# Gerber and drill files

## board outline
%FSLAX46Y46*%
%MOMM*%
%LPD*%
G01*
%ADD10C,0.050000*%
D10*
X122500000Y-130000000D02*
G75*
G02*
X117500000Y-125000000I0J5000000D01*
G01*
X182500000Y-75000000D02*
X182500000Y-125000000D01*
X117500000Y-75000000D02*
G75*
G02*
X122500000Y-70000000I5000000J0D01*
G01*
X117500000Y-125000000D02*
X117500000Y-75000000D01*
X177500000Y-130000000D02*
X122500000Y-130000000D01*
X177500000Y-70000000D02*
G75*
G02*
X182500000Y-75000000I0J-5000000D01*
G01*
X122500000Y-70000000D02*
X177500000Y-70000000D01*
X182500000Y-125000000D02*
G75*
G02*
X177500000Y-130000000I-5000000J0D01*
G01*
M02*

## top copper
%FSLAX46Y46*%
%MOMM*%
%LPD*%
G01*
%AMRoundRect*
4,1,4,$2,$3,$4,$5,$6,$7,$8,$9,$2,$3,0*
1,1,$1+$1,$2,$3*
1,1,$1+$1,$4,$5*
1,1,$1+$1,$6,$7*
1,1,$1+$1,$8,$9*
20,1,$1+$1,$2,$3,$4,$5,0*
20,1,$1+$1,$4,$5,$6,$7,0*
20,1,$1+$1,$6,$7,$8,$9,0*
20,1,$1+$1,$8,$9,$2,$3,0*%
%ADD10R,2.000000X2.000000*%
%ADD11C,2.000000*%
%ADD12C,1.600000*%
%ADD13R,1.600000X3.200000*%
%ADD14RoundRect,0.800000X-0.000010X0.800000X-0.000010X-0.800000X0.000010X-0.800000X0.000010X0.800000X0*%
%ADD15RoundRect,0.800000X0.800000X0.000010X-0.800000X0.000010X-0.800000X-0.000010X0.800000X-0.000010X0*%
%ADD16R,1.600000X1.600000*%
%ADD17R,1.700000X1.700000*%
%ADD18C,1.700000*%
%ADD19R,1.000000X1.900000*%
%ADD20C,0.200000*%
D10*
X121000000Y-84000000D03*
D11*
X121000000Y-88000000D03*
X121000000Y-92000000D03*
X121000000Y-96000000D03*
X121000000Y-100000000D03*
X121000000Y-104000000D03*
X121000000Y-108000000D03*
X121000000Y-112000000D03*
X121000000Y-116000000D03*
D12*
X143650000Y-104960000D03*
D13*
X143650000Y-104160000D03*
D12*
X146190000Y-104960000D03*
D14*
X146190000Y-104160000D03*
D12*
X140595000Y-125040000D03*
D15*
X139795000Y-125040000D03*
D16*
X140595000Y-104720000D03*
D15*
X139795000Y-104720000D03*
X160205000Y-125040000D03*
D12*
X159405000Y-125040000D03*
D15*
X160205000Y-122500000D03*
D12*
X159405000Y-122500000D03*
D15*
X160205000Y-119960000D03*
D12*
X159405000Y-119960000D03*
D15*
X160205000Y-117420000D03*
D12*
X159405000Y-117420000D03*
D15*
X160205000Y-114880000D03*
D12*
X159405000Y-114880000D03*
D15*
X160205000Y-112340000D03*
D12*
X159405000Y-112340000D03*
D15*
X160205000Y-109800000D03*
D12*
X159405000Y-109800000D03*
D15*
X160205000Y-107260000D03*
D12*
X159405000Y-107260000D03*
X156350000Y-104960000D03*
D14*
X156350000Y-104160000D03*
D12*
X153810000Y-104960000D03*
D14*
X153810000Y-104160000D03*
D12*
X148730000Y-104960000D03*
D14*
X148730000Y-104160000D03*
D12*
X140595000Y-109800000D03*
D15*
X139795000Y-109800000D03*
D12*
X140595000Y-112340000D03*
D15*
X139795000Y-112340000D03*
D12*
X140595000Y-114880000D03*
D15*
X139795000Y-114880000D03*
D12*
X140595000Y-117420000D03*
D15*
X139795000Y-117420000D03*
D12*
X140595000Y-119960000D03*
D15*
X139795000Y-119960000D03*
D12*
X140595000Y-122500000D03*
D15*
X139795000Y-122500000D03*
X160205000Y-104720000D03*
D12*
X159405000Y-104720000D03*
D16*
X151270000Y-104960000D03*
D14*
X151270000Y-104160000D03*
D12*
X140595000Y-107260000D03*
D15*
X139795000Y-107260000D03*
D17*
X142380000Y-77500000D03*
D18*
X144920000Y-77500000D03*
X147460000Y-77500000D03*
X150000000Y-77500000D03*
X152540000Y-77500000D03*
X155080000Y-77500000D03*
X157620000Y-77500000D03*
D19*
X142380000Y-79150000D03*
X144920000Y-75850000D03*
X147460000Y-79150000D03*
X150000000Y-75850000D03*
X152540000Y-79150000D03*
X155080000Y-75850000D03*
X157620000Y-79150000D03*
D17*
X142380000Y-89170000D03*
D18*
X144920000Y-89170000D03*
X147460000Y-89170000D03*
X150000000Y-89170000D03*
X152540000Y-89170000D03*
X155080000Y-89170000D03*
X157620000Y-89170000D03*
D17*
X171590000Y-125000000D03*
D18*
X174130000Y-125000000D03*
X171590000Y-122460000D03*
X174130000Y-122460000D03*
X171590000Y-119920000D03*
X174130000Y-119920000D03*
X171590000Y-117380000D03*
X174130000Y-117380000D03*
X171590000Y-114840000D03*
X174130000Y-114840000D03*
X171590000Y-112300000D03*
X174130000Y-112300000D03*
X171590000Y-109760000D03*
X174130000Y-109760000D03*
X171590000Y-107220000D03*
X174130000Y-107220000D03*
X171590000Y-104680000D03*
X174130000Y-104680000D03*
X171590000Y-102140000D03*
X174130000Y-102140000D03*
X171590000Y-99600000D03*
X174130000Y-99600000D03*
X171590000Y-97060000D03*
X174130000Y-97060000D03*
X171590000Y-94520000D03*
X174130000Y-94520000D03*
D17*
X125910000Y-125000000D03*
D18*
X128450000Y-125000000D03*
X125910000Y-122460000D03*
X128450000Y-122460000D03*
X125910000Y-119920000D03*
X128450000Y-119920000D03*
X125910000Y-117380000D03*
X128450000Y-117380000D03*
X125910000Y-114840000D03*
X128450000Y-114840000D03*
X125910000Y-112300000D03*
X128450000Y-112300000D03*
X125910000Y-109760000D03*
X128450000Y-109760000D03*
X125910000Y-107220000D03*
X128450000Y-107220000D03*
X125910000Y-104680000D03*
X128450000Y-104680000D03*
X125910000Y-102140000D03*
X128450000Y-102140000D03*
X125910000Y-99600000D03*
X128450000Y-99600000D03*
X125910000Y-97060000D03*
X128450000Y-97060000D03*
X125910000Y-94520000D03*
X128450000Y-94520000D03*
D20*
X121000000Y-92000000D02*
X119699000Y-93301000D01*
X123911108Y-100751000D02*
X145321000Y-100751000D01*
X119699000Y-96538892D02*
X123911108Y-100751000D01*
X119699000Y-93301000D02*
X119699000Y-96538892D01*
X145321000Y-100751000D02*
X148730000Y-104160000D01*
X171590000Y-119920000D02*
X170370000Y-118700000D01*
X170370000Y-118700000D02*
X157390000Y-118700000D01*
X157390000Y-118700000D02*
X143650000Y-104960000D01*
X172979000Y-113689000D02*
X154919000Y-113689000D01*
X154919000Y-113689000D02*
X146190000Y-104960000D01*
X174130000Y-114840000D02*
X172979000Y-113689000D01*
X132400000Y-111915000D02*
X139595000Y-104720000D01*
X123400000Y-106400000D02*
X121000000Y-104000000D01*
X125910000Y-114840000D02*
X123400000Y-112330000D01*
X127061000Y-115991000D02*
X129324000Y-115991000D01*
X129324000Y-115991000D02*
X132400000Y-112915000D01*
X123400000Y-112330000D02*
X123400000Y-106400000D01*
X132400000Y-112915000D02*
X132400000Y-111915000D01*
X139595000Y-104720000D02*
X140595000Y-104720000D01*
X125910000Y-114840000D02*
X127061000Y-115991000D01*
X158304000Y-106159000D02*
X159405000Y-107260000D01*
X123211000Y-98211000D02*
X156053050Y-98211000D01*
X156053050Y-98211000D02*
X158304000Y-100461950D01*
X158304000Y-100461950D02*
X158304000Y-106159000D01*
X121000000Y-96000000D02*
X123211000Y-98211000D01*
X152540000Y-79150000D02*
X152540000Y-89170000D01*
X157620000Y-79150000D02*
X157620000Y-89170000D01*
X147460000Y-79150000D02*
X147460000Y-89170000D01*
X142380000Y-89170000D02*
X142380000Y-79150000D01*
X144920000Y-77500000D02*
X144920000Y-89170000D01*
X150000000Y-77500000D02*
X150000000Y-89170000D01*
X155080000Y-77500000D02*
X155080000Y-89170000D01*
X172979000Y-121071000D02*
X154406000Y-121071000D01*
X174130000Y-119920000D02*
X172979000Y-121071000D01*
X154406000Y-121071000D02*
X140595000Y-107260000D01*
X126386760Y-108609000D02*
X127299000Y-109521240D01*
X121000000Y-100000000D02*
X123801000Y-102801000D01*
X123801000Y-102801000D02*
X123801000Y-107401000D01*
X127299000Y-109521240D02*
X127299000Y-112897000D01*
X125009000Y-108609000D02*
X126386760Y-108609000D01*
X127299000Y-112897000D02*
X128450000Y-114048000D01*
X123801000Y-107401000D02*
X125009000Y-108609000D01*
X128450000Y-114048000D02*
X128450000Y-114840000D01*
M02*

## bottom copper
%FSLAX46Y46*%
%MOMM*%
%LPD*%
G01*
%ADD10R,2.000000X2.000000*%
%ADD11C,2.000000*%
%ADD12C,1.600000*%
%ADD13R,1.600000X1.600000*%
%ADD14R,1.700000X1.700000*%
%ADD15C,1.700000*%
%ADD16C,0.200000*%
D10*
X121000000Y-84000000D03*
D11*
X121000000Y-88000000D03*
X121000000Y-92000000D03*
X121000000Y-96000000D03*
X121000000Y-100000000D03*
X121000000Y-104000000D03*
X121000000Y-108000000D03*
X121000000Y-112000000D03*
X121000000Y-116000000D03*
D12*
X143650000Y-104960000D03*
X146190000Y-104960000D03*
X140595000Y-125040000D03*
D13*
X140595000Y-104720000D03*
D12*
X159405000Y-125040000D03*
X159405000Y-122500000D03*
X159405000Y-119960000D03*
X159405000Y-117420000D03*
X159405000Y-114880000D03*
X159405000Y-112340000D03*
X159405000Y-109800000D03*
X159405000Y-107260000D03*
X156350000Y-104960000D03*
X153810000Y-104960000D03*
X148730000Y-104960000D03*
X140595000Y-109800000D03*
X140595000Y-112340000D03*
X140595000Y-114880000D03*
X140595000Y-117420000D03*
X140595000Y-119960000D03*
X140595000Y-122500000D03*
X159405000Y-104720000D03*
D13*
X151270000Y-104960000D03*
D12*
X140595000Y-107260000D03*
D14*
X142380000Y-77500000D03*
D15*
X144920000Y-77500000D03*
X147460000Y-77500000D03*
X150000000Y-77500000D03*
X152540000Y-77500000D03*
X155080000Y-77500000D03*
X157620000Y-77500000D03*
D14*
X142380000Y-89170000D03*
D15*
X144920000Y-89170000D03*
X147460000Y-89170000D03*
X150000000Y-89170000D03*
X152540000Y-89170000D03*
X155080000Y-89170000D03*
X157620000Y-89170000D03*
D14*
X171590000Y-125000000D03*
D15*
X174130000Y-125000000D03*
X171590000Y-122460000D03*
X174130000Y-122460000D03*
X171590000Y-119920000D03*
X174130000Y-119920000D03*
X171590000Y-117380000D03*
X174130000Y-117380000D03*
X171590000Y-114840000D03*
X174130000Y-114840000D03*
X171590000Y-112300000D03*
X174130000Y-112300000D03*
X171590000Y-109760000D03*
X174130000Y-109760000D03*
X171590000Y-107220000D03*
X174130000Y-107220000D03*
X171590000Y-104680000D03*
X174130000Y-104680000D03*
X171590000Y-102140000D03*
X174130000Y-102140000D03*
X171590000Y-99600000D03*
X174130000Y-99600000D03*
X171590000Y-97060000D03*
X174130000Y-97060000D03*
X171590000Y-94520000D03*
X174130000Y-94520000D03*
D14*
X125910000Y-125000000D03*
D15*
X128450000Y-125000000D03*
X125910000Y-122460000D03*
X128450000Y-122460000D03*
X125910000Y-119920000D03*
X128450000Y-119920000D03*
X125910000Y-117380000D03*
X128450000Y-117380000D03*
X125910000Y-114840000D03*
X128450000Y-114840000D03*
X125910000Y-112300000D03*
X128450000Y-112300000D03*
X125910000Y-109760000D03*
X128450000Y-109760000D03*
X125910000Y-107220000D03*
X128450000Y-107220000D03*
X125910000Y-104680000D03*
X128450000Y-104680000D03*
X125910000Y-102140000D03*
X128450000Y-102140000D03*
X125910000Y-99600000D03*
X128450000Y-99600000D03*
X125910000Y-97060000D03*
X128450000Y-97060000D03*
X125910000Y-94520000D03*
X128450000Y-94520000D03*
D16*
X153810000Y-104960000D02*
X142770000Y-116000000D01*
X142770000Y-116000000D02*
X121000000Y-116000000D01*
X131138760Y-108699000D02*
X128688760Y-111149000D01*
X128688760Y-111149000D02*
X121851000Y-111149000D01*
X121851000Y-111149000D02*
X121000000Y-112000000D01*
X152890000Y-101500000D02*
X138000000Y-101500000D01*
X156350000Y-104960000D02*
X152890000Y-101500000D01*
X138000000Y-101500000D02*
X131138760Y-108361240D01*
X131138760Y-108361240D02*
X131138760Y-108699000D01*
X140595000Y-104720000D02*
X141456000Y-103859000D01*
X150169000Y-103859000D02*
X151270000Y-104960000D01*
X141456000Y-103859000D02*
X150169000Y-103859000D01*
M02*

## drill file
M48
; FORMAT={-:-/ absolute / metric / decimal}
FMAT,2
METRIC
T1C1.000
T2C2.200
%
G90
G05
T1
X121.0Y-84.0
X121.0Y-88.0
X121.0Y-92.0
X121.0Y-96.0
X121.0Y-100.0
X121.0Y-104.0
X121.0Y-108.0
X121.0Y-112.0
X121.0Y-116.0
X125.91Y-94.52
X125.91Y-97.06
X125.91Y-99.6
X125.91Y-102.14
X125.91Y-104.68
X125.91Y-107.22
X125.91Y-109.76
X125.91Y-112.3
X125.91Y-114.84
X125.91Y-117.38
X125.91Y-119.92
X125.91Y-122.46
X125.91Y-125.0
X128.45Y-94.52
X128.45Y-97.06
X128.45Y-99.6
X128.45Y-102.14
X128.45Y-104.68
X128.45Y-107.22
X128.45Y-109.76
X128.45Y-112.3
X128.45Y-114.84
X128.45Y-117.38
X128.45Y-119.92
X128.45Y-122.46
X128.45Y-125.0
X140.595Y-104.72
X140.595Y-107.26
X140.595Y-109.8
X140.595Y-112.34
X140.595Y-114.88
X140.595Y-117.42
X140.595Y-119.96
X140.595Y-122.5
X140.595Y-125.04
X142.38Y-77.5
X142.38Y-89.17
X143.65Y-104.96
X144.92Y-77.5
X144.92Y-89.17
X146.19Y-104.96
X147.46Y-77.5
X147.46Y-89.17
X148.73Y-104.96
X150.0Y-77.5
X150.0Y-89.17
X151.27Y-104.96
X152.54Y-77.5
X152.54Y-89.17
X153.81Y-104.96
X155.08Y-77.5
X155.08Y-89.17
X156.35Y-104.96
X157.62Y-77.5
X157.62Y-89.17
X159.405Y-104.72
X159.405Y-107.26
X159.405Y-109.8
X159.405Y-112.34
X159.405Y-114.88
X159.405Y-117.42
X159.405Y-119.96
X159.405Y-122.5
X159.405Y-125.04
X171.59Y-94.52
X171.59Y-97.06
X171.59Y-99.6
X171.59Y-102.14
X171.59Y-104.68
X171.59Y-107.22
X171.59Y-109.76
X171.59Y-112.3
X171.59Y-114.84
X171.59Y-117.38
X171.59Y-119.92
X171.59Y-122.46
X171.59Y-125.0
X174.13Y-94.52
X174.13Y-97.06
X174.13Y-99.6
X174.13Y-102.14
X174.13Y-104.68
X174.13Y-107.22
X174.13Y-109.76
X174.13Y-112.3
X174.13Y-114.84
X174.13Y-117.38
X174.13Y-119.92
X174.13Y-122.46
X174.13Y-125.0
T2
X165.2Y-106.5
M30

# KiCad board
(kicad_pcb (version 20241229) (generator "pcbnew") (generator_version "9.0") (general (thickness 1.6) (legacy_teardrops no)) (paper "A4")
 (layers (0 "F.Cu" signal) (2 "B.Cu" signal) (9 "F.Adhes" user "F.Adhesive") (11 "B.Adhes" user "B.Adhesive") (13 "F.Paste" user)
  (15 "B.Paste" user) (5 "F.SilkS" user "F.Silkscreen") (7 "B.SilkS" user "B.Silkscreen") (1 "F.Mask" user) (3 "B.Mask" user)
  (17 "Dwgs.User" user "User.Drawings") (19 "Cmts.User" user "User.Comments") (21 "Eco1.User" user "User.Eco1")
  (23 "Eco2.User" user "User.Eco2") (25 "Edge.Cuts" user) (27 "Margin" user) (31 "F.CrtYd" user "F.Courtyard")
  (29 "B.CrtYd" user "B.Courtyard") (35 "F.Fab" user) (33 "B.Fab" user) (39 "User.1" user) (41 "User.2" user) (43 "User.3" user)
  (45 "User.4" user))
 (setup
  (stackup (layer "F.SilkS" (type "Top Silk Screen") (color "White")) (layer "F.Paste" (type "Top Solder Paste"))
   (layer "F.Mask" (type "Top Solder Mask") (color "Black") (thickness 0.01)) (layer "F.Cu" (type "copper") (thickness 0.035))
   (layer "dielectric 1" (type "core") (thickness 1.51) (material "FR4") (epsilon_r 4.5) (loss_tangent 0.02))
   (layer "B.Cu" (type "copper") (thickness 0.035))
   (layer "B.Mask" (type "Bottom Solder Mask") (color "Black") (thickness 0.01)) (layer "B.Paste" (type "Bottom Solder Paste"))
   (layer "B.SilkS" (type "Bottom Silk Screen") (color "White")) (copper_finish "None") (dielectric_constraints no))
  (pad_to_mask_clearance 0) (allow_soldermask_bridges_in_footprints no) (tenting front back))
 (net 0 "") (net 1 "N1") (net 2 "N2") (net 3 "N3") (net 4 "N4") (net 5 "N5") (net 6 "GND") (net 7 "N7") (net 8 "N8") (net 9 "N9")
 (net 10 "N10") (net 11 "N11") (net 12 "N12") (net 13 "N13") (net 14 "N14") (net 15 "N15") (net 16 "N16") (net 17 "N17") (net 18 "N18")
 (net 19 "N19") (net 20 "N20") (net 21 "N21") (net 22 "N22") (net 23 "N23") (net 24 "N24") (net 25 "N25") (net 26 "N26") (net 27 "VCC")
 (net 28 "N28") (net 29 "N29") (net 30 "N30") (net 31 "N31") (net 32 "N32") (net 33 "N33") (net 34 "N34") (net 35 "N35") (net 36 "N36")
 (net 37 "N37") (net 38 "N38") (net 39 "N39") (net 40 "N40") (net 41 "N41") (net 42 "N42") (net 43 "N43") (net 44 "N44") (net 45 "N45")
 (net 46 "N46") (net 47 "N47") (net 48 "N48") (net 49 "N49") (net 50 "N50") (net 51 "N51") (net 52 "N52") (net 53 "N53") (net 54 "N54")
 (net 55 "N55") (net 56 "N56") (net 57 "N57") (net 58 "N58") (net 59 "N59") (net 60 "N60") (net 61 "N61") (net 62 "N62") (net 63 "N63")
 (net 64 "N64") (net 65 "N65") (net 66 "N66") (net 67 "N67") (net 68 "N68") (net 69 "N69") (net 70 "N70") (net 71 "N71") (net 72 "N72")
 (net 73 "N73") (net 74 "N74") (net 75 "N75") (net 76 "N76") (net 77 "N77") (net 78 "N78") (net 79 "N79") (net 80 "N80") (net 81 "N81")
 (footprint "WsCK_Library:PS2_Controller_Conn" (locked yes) (layer "F.Cu") (at 121 100)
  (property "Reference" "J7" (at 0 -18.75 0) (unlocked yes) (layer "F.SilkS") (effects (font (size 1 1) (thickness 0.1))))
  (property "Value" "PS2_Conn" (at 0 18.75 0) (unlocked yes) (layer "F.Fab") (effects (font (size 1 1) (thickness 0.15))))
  (pad "1" thru_hole rect (at 0 -16 270) (size 2 2) (drill 1) (layers "*.Cu" "*.Mask") (remove_unused_layers no) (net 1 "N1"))
  (pad "2" thru_hole circle (at 0 -12 270) (size 2 2) (drill 1) (layers "*.Cu" "*.Mask") (remove_unused_layers no) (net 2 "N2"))
  (pad "3" thru_hole circle (at 0 -8 270) (size 2 2) (drill 1) (layers "*.Cu" "*.Mask") (remove_unused_layers no) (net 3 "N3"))
  (pad "4" thru_hole circle (at 0 -4 270) (size 2 2) (drill 1) (layers "*.Cu" "*.Mask") (remove_unused_layers no) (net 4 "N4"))
  (pad "5" thru_hole circle (at 0 0 270) (size 2 2) (drill 1) (layers "*.Cu" "*.Mask") (remove_unused_layers no) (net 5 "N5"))
  (pad "6" thru_hole circle (at 0 4 270) (size 2 2) (drill 1) (layers "*.Cu" "*.Mask") (remove_unused_layers no) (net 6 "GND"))
  (pad "7" thru_hole circle (at 0 8 270) (size 2 2) (drill 1) (layers "*.Cu" "*.Mask") (remove_unused_layers no) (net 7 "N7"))
  (pad "8" thru_hole circle (at 0 12 270) (size 2 2) (drill 1) (layers "*.Cu" "*.Mask") (remove_unused_layers no) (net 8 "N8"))
  (pad "9" thru_hole circle (at 0 16 270) (size 2 2) (drill 1) (layers "*.Cu" "*.Mask") (remove_unused_layers no) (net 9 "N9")))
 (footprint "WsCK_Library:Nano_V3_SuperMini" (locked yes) (layer "F.Cu") (at 150 116.66 180)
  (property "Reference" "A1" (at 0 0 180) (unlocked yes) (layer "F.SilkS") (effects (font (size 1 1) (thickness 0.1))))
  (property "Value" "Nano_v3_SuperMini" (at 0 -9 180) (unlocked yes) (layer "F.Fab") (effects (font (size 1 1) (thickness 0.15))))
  (pad "1" thru_hole circle (at 6.35 11.7 180) (size 1.6 1.6) (drill 1) (layers "*.Cu" "*.Mask") (remove_unused_layers no) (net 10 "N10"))
  (pad "1" smd rect (at 6.35 12.5 270) (size 3.2 1.6) (layers "F.Cu" "F.Mask") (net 10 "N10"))
  (pad "2" thru_hole circle (at 3.81 11.7 180) (size 1.6 1.6) (drill 1) (layers "*.Cu" "*.Mask") (remove_unused_layers no) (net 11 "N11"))
  (pad "2" smd roundrect (at 3.81 12.5 270) (size 3.2 1.6) (layers "F.Cu" "F.Mask") (roundrect_rratio 0.5) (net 11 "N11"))
  (pad "3" thru_hole circle (at 9.405 -8.38 180) (size 1.6 1.6) (drill 1) (layers "*.Cu" "*.Mask") (remove_unused_layers no) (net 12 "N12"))
  (pad "3" smd roundrect (at 10.205 -8.38 180) (size 3.2 1.6) (layers "F.Cu" "F.Mask") (roundrect_rratio 0.5) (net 12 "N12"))
  (pad "4" thru_hole rect (at 9.405 11.94 180) (size 1.6 1.6) (drill 1) (layers "*.Cu" "*.Mask") (remove_unused_layers no) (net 6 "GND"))
  (pad "4" smd roundrect (at 10.205 11.94 180) (size 3.2 1.6) (layers "F.Cu" "F.Mask") (roundrect_rratio 0.5) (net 6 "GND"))
  (pad "6" smd roundrect (at -10.205 -8.38 180) (size 3.2 1.6) (layers "F.Cu" "F.Mask") (roundrect_rratio 0.5) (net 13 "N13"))
  (pad "6" thru_hole circle (at -9.405 -8.38 180) (size 1.6 1.6) (drill 1) (layers "*.Cu" "*.Mask") (remove_unused_layers no) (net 13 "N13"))
  (pad "7" smd roundrect (at -10.205 -5.84 180) (size 3.2 1.6) (layers "F.Cu" "F.Mask") (roundrect_rratio 0.5) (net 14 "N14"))
  (pad "7" thru_hole circle (at -9.405 -5.84 180) (size 1.6 1.6) (drill 1) (layers "*.Cu" "*.Mask") (remove_unused_layers no) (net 14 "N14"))
  (pad "8" smd roundrect (at -10.205 -3.3 180) (size 3.2 1.6) (layers "F.Cu" "F.Mask") (roundrect_rratio 0.5) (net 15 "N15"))
  (pad "8" thru_hole circle (at -9.405 -3.3 180) (size 1.6 1.6) (drill 1) (layers "*.Cu" "*.Mask") (remove_unused_layers no) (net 15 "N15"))
  (pad "9" smd roundrect (at -10.205 -0.76 180) (size 3.2 1.6) (layers "F.Cu" "F.Mask") (roundrect_rratio 0.5) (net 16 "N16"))
  (pad "9" thru_hole circle (at -9.405 -0.76 180) (size 1.6 1.6) (drill 1) (layers "*.Cu" "*.Mask") (remove_unused_layers no) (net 16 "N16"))
  (pad "10" smd roundrect (at -10.205 1.78 180) (size 3.2 1.6) (layers "F.Cu" "F.Mask") (roundrect_rratio 0.5) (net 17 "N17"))
  (pad "10" thru_hole circle (at -9.405 1.78 180) (size 1.6 1.6) (drill 1) (layers "*.Cu" "*.Mask") (remove_unused_layers no) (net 17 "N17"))
  (pad "11" smd roundrect (at -10.205 4.32 180) (size 3.2 1.6) (layers "F.Cu" "F.Mask") (roundrect_rratio 0.5) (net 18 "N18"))
  (pad "11" thru_hole circle (at -9.405 4.32 180) (size 1.6 1.6) (drill 1) (layers "*.Cu" "*.Mask") (remove_unused_layers no) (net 18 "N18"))
  (pad "12" smd roundrect (at -10.205 6.86 180) (size 3.2 1.6) (layers "F.Cu" "F.Mask") (roundrect_rratio 0.5) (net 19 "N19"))
  (pad "12" thru_hole circle (at -9.405 6.86 180) (size 1.6 1.6) (drill 1) (layers "*.Cu" "*.Mask") (remove_unused_layers no) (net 19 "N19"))
  (pad "13" smd roundrect (at -10.205 9.4 180) (size 3.2 1.6) (layers "F.Cu" "F.Mask") (roundrect_rratio 0.5) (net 4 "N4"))
  (pad "13" thru_hole circle (at -9.405 9.4 180) (size 1.6 1.6) (drill 1) (layers "*.Cu" "*.Mask") (remove_unused_layers no) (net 4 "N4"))
  (pad "14" thru_hole circle (at -6.35 11.7 180) (size 1.6 1.6) (drill 1) (layers "*.Cu" "*.Mask") (remove_unused_layers no) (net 8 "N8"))
  (pad "14" smd roundrect (at -6.35 12.5 270) (size 3.2 1.6) (layers "F.Cu" "F.Mask") (roundrect_rratio 0.5) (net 8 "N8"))
  (pad "15" thru_hole circle (at -3.81 11.7 180) (size 1.6 1.6) (drill 1) (layers "*.Cu" "*.Mask") (remove_unused_layers no) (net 9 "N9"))
  (pad "15" smd roundrect (at -3.81 12.5 270) (size 3.2 1.6) (layers "F.Cu" "F.Mask") (roundrect_rratio 0.5) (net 9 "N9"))
  (pad "16" thru_hole circle (at 1.27 11.7 180) (size 1.6 1.6) (drill 1) (layers "*.Cu" "*.Mask") (remove_unused_layers no) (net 3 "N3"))
  (pad "16" smd roundrect (at 1.27 12.5 270) (size 3.2 1.6) (layers "F.Cu" "F.Mask") (roundrect_rratio 0.5) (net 3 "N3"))
  (pad "19" thru_hole circle (at 9.405 6.86 180) (size 1.6 1.6) (drill 1) (layers "*.Cu" "*.Mask") (remove_unused_layers no) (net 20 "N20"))
  (pad "19" smd roundrect (at 10.205 6.86 180) (size 3.2 1.6) (layers "F.Cu" "F.Mask") (roundrect_rratio 0.5) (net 20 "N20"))
  (pad "20" thru_hole circle (at 9.405 4.32 180) (size 1.6 1.6) (drill 1) (layers "*.Cu" "*.Mask") (remove_unused_layers no) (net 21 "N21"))
  (pad "20" smd roundrect (at 10.205 4.32 180) (size 3.2 1.6) (layers "F.Cu" "F.Mask") (roundrect_rratio 0.5) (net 21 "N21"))
  (pad "21" thru_hole circle (at 9.405 1.78 180) (size 1.6 1.6) (drill 1) (layers "*.Cu" "*.Mask") (remove_unused_layers no) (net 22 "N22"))
  (pad "21" smd roundrect (at 10.205 1.78 180) (size 3.2 1.6) (layers "F.Cu" "F.Mask") (roundrect_rratio 0.5) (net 22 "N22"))
  (pad "22" thru_hole circle (at 9.405 -0.76 180) (size 1.6 1.6) (drill 1) (layers "*.Cu" "*.Mask") (remove_unused_layers no) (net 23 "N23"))
  (pad "22" smd roundrect (at 10.205 -0.76 180) (size 3.2 1.6) (layers "F.Cu" "F.Mask") (roundrect_rratio 0.5) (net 23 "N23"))
  (pad "23" thru_hole circle (at 9.405 -3.3 180) (size 1.6 1.6) (drill 1) (layers "*.Cu" "*.Mask") (remove_unused_layers no) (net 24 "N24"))
  (pad "23" smd roundrect (at 10.205 -3.3 180) (size 3.2 1.6) (layers "F.Cu" "F.Mask") (roundrect_rratio 0.5) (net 24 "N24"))
  (pad "24" thru_hole circle (at 9.405 -5.84 180) (size 1.6 1.6) (drill 1) (layers "*.Cu" "*.Mask") (remove_unused_layers no) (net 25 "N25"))
  (pad "24" smd roundrect (at 10.205 -5.84 180) (size 3.2 1.6) (layers "F.Cu" "F.Mask") (roundrect_rratio 0.5) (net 25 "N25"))
  (pad "27" smd roundrect (at -10.205 11.94 180) (size 3.2 1.6) (layers "F.Cu" "F.Mask") (roundrect_rratio 0.5) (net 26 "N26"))
  (pad "27" thru_hole circle (at -9.405 11.94 180) (size 1.6 1.6) (drill 1) (layers "*.Cu" "*.Mask") (remove_unused_layers no)
   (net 26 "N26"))
  (pad "29" thru_hole rect (at -1.27 11.7 180) (size 1.6 1.6) (drill 1) (layers "*.Cu" "*.Mask") (remove_unused_layers no) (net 6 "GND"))
  (pad "29" smd roundrect (at -1.27 12.5 270) (size 3.2 1.6) (layers "F.Cu" "F.Mask") (roundrect_rratio 0.5) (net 6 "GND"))
  (pad "30" thru_hole circle (at 9.405 9.4 180) (size 1.6 1.6) (drill 1) (layers "*.Cu" "*.Mask") (remove_unused_layers no) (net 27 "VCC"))
  (pad "30" smd roundrect (at 10.205 9.4 180) (size 3.2 1.6) (layers "F.Cu" "F.Mask") (roundrect_rratio 0.5) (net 27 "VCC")))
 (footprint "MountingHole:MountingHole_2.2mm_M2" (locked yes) (layer "F.Cu") (at 165.2 106.5)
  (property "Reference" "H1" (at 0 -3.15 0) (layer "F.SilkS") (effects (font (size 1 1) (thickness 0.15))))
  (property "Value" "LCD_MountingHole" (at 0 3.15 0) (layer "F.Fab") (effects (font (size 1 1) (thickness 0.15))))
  (pad "" np_thru_hole circle (at 0 0) (size 2.2 2.2) (drill 2.2) (layers "*.Cu" "*.Mask")))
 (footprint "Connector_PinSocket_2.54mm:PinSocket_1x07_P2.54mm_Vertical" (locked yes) (layer "F.Cu") (at 142.38 77.5 90)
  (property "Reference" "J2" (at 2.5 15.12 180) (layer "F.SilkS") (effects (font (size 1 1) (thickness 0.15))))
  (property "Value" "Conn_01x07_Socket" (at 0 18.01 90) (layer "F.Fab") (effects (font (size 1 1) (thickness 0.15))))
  (pad "1" thru_hole rect (at 0 0 90) (size 1.7 1.7) (drill 1) (layers "*.Cu" "*.Mask") (remove_unused_layers no) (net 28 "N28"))
  (pad "2" thru_hole circle (at 0 2.54 90) (size 1.7 1.7) (drill 1) (layers "*.Cu" "*.Mask") (remove_unused_layers no) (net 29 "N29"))
  (pad "3" thru_hole circle (at 0 5.08 90) (size 1.7 1.7) (drill 1) (layers "*.Cu" "*.Mask") (remove_unused_layers no) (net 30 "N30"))
  (pad "4" thru_hole circle (at 0 7.62 90) (size 1.7 1.7) (drill 1) (layers "*.Cu" "*.Mask") (remove_unused_layers no) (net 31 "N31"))
  (pad "5" thru_hole circle (at 0 10.16 90) (size 1.7 1.7) (drill 1) (layers "*.Cu" "*.Mask") (remove_unused_layers no) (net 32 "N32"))
  (pad "6" thru_hole circle (at 0 12.7 90) (size 1.7 1.7) (drill 1) (layers "*.Cu" "*.Mask") (remove_unused_layers no) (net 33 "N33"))
  (pad "7" thru_hole circle (at 0 15.24 90) (size 1.7 1.7) (drill 1) (layers "*.Cu" "*.Mask") (remove_unused_layers no) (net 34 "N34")))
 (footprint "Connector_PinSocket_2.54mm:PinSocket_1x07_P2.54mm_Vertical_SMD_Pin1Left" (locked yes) (layer "F.Cu") (at 150 77.5 90)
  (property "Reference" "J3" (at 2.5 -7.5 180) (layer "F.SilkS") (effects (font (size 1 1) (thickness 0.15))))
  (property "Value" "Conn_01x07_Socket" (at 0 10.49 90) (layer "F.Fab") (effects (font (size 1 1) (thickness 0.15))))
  (pad "1" smd rect (at -1.65 -7.62 90) (size 1.9 1) (layers "F.Cu" "F.Mask" "F.Paste") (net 28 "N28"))
  (pad "2" smd rect (at 1.65 -5.08 90) (size 1.9 1) (layers "F.Cu" "F.Mask" "F.Paste") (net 29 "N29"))
  (pad "3" smd rect (at -1.65 -2.54 90) (size 1.9 1) (layers "F.Cu" "F.Mask" "F.Paste") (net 30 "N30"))
  (pad "4" smd rect (at 1.65 0 90) (size 1.9 1) (layers "F.Cu" "F.Mask" "F.Paste") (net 31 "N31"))
  (pad "5" smd rect (at -1.65 2.54 90) (size 1.9 1) (layers "F.Cu" "F.Mask" "F.Paste") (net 32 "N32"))
  (pad "6" smd rect (at 1.65 5.08 90) (size 1.9 1) (layers "F.Cu" "F.Mask" "F.Paste") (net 33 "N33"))
  (pad "7" smd rect (at -1.65 7.62 90) (size 1.9 1) (layers "F.Cu" "F.Mask" "F.Paste") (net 34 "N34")))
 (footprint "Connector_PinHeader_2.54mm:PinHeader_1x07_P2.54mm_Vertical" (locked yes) (layer "B.Cu") (at 142.38 89.17 -90)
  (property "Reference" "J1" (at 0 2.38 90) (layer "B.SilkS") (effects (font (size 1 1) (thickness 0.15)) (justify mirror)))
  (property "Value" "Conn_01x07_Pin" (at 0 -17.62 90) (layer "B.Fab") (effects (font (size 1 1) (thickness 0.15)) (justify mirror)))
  (pad "1" thru_hole rect (at 0 0 270) (size 1.7 1.7) (drill 1) (layers "*.Cu" "*.Mask") (remove_unused_layers no) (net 28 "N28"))
  (pad "2" thru_hole circle (at 0 -2.54 270) (size 1.7 1.7) (drill 1) (layers "*.Cu" "*.Mask") (remove_unused_layers no) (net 29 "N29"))
  (pad "3" thru_hole circle (at 0 -5.08 270) (size 1.7 1.7) (drill 1) (layers "*.Cu" "*.Mask") (remove_unused_layers no) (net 30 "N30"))
  (pad "4" thru_hole circle (at 0 -7.62 270) (size 1.7 1.7) (drill 1) (layers "*.Cu" "*.Mask") (remove_unused_layers no) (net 31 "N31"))
  (pad "5" thru_hole circle (at 0 -10.16 270) (size 1.7 1.7) (drill 1) (layers "*.Cu" "*.Mask") (remove_unused_layers no) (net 32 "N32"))
  (pad "6" thru_hole circle (at 0 -12.7 270) (size 1.7 1.7) (drill 1) (layers "*.Cu" "*.Mask") (remove_unused_layers no) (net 33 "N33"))
  (pad "7" thru_hole circle (at 0 -15.24 270) (size 1.7 1.7) (drill 1) (layers "*.Cu" "*.Mask") (remove_unused_layers no) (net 34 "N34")))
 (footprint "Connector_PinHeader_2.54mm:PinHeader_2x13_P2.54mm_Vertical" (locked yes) (layer "B.Cu") (at 171.59 125)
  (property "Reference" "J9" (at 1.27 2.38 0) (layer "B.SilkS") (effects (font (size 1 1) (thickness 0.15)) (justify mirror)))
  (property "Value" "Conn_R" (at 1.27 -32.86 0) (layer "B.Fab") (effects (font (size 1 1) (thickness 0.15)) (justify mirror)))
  (pad "1" thru_hole rect (at 0 0) (size 1.7 1.7) (drill 1) (layers "*.Cu" "*.Mask") (remove_unused_layers no) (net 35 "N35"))
  (pad "2" thru_hole circle (at 2.54 0) (size 1.7 1.7) (drill 1) (layers "*.Cu" "*.Mask") (remove_unused_layers no) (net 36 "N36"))
  (pad "3" thru_hole circle (at 0 -2.54) (size 1.7 1.7) (drill 1) (layers "*.Cu" "*.Mask") (remove_unused_layers no) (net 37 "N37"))
  (pad "4" thru_hole circle (at 2.54 -2.54) (size 1.7 1.7) (drill 1) (layers "*.Cu" "*.Mask") (remove_unused_layers no) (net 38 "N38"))
  (pad "5" thru_hole circle (at 0 -5.08) (size 1.7 1.7) (drill 1) (layers "*.Cu" "*.Mask") (remove_unused_layers no) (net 10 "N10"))
  (pad "6" thru_hole circle (at 2.54 -5.08) (size 1.7 1.7) (drill 1) (layers "*.Cu" "*.Mask") (remove_unused_layers no) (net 27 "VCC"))
  (pad "7" thru_hole circle (at 0 -7.62) (size 1.7 1.7) (drill 1) (layers "*.Cu" "*.Mask") (remove_unused_layers no) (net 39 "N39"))
  (pad "8" thru_hole circle (at 2.54 -7.62) (size 1.7 1.7) (drill 1) (layers "*.Cu" "*.Mask") (remove_unused_layers no) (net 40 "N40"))
  (pad "9" thru_hole circle (at 0 -10.16) (size 1.7 1.7) (drill 1) (layers "*.Cu" "*.Mask") (remove_unused_layers no) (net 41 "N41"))
  (pad "10" thru_hole circle (at 2.54 -10.16) (size 1.7 1.7) (drill 1) (layers "*.Cu" "*.Mask") (remove_unused_layers no) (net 11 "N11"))
  (pad "11" thru_hole circle (at 0 -12.7) (size 1.7 1.7) (drill 1) (layers "*.Cu" "*.Mask") (remove_unused_layers no) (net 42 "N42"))
  (pad "12" thru_hole circle (at 2.54 -12.7) (size 1.7 1.7) (drill 1) (layers "*.Cu" "*.Mask") (remove_unused_layers no) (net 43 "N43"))
  (pad "13" thru_hole circle (at 0 -15.24) (size 1.7 1.7) (drill 1) (layers "*.Cu" "*.Mask") (remove_unused_layers no) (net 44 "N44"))
  (pad "14" thru_hole circle (at 2.54 -15.24) (size 1.7 1.7) (drill 1) (layers "*.Cu" "*.Mask") (remove_unused_layers no) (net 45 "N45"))
  (pad "15" thru_hole circle (at 0 -17.78) (size 1.7 1.7) (drill 1) (layers "*.Cu" "*.Mask") (remove_unused_layers no) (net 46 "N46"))
  (pad "16" thru_hole circle (at 2.54 -17.78) (size 1.7 1.7) (drill 1) (layers "*.Cu" "*.Mask") (remove_unused_layers no) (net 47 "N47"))
  (pad "17" thru_hole circle (at 0 -20.32) (size 1.7 1.7) (drill 1) (layers "*.Cu" "*.Mask") (remove_unused_layers no) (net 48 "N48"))
  (pad "18" thru_hole circle (at 2.54 -20.32) (size 1.7 1.7) (drill 1) (layers "*.Cu" "*.Mask") (remove_unused_layers no) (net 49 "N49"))
  (pad "19" thru_hole circle (at 0 -22.86) (size 1.7 1.7) (drill 1) (layers "*.Cu" "*.Mask") (remove_unused_layers no) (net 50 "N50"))
  (pad "20" thru_hole circle (at 2.54 -22.86) (size 1.7 1.7) (drill 1) (layers "*.Cu" "*.Mask") (remove_unused_layers no) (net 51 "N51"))
  (pad "21" thru_hole circle (at 0 -25.4) (size 1.7 1.7) (drill 1) (layers "*.Cu" "*.Mask") (remove_unused_layers no) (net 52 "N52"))
  (pad "22" thru_hole circle (at 2.54 -25.4) (size 1.7 1.7) (drill 1) (layers "*.Cu" "*.Mask") (remove_unused_layers no) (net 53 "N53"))
  (pad "23" thru_hole circle (at 0 -27.94) (size 1.7 1.7) (drill 1) (layers "*.Cu" "*.Mask") (remove_unused_layers no) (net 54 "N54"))
  (pad "24" thru_hole circle (at 2.54 -27.94) (size 1.7 1.7) (drill 1) (layers "*.Cu" "*.Mask") (remove_unused_layers no) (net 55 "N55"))
  (pad "25" thru_hole circle (at 0 -30.48) (size 1.7 1.7) (drill 1) (layers "*.Cu" "*.Mask") (remove_unused_layers no) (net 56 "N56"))
  (pad "26" thru_hole circle (at 2.54 -30.48) (size 1.7 1.7) (drill 1) (layers "*.Cu" "*.Mask") (remove_unused_layers no) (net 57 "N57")))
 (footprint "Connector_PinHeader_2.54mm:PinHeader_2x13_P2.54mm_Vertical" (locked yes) (layer "B.Cu") (at 125.91 125)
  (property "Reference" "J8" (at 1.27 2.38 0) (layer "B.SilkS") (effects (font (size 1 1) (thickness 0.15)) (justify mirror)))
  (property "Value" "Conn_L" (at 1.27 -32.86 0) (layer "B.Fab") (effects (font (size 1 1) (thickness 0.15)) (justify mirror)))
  (pad "1" thru_hole rect (at 0 0) (size 1.7 1.7) (drill 1) (layers "*.Cu" "*.Mask") (remove_unused_layers no) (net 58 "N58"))
  (pad "2" thru_hole circle (at 2.54 0) (size 1.7 1.7) (drill 1) (layers "*.Cu" "*.Mask") (remove_unused_layers no) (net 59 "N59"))
  (pad "3" thru_hole circle (at 0 -2.54) (size 1.7 1.7) (drill 1) (layers "*.Cu" "*.Mask") (remove_unused_layers no) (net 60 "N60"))
  (pad "4" thru_hole circle (at 2.54 -2.54) (size 1.7 1.7) (drill 1) (layers "*.Cu" "*.Mask") (remove_unused_layers no) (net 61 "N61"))
  (pad "5" thru_hole circle (at 0 -5.08) (size 1.7 1.7) (drill 1) (layers "*.Cu" "*.Mask") (remove_unused_layers no) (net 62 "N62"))
  (pad "6" thru_hole circle (at 2.54 -5.08) (size 1.7 1.7) (drill 1) (layers "*.Cu" "*.Mask") (remove_unused_layers no) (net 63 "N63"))
  (pad "7" thru_hole circle (at 0 -7.62) (size 1.7 1.7) (drill 1) (layers "*.Cu" "*.Mask") (remove_unused_layers no) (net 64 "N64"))
  (pad "8" thru_hole circle (at 2.54 -7.62) (size 1.7 1.7) (drill 1) (layers "*.Cu" "*.Mask") (remove_unused_layers no) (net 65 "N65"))
  (pad "9" thru_hole circle (at 0 -10.16) (size 1.7 1.7) (drill 1) (layers "*.Cu" "*.Mask") (remove_unused_layers no) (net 6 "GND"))
  (pad "10" thru_hole circle (at 2.54 -10.16) (size 1.7 1.7) (drill 1) (layers "*.Cu" "*.Mask") (remove_unused_layers no) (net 5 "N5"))
  (pad "11" thru_hole circle (at 0 -12.7) (size 1.7 1.7) (drill 1) (layers "*.Cu" "*.Mask") (remove_unused_layers no) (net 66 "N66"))
  (pad "12" thru_hole circle (at 2.54 -12.7) (size 1.7 1.7) (drill 1) (layers "*.Cu" "*.Mask") (remove_unused_layers no) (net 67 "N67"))
  (pad "13" thru_hole circle (at 0 -15.24) (size 1.7 1.7) (drill 1) (layers "*.Cu" "*.Mask") (remove_unused_layers no) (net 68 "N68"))
  (pad "14" thru_hole circle (at 2.54 -15.24) (size 1.7 1.7) (drill 1) (layers "*.Cu" "*.Mask") (remove_unused_layers no) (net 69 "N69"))
  (pad "15" thru_hole circle (at 0 -17.78) (size 1.7 1.7) (drill 1) (layers "*.Cu" "*.Mask") (remove_unused_layers no) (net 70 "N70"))
  (pad "16" thru_hole circle (at 2.54 -17.78) (size 1.7 1.7) (drill 1) (layers "*.Cu" "*.Mask") (remove_unused_layers no) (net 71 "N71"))
  (pad "17" thru_hole circle (at 0 -20.32) (size 1.7 1.7) (drill 1) (layers "*.Cu" "*.Mask") (remove_unused_layers no) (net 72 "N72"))
  (pad "18" thru_hole circle (at 2.54 -20.32) (size 1.7 1.7) (drill 1) (layers "*.Cu" "*.Mask") (remove_unused_layers no) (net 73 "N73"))
  (pad "19" thru_hole circle (at 0 -22.86) (size 1.7 1.7) (drill 1) (layers "*.Cu" "*.Mask") (remove_unused_layers no) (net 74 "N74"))
  (pad "20" thru_hole circle (at 2.54 -22.86) (size 1.7 1.7) (drill 1) (layers "*.Cu" "*.Mask") (remove_unused_layers no) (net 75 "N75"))
  (pad "21" thru_hole circle (at 0 -25.4) (size 1.7 1.7) (drill 1) (layers "*.Cu" "*.Mask") (remove_unused_layers no) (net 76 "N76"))
  (pad "22" thru_hole circle (at 2.54 -25.4) (size 1.7 1.7) (drill 1) (layers "*.Cu" "*.Mask") (remove_unused_layers no) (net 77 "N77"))
  (pad "23" thru_hole circle (at 0 -27.94) (size 1.7 1.7) (drill 1) (layers "*.Cu" "*.Mask") (remove_unused_layers no) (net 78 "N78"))
  (pad "24" thru_hole circle (at 2.54 -27.94) (size 1.7 1.7) (drill 1) (layers "*.Cu" "*.Mask") (remove_unused_layers no) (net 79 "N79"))
  (pad "25" thru_hole circle (at 0 -30.48) (size 1.7 1.7) (drill 1) (layers "*.Cu" "*.Mask") (remove_unused_layers no) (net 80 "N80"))
  (pad "26" thru_hole circle (at 2.54 -30.48) (size 1.7 1.7) (drill 1) (layers "*.Cu" "*.Mask") (remove_unused_layers no) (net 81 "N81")))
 (gr_arc (start 122.5 130) (mid 118.964466 128.535534) (end 117.5 125) (stroke (width 0.05) (type default)) (layer "Edge.Cuts"))
 (gr_line (start 182.5 75) (end 182.5 125) (stroke (width 0.05) (type default)) (layer "Edge.Cuts"))
 (gr_arc (start 117.5 75) (mid 118.964466 71.464466) (end 122.5 70) (stroke (width 0.05) (type default)) (layer "Edge.Cuts"))
 (gr_line (start 117.5 125) (end 117.5 75) (stroke (width 0.05) (type default)) (layer "Edge.Cuts"))
 (gr_line (start 177.5 130) (end 122.5 130) (stroke (width 0.05) (type default)) (layer "Edge.Cuts"))
 (gr_arc (start 177.5 70) (mid 181.035534 71.464466) (end 182.5 75) (stroke (width 0.05) (type default)) (layer "Edge.Cuts"))
 (gr_line (start 122.5 70) (end 177.5 70) (stroke (width 0.05) (type default)) (layer "Edge.Cuts"))
 (gr_arc (start 182.5 125) (mid 181.035534 128.535534) (end 177.5 130) (stroke (width 0.05) (type default)) (layer "Edge.Cuts"))
 (segment (start 121 92) (end 119.699 93.301) (width 0.2) (layer "F.Cu") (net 3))
 (segment (start 123.911108 100.751) (end 145.321 100.751) (width 0.2) (layer "F.Cu") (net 3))
 (segment (start 119.699 96.538892) (end 123.911108 100.751) (width 0.2) (layer "F.Cu") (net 3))
 (segment (start 119.699 93.301) (end 119.699 96.538892) (width 0.2) (layer "F.Cu") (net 3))
 (segment (start 145.321 100.751) (end 148.73 104.16) (width 0.2) (layer "F.Cu") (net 3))
 (segment (start 171.59 119.92) (end 170.37 118.7) (width 0.2) (layer "F.Cu") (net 10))
 (segment (start 170.37 118.7) (end 157.39 118.7) (width 0.2) (layer "F.Cu") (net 10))
 (segment (start 157.39 118.7) (end 143.65 104.96) (width 0.2) (layer "F.Cu") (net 10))
 (segment (start 153.81 104.96) (end 142.77 116) (width 0.2) (layer "B.Cu") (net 9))
 (segment (start 142.77 116) (end 121 116) (width 0.2) (layer "B.Cu") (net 9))
 (segment (start 131.13876 108.699) (end 128.68876 111.149) (width 0.2) (layer "B.Cu") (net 8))
 (segment (start 128.68876 111.149) (end 121.851 111.149) (width 0.2) (layer "B.Cu") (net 8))
 (segment (start 121.851 111.149) (end 121 112) (width 0.2) (layer "B.Cu") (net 8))
 (segment (start 152.89 101.5) (end 138 101.5) (width 0.2) (layer "B.Cu") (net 8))
 (segment (start 156.35 104.96) (end 152.89 101.5) (width 0.2) (layer "B.Cu") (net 8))
 (segment (start 138 101.5) (end 131.13876 108.36124) (width 0.2) (layer "B.Cu") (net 8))
 (segment (start 131.13876 108.36124) (end 131.13876 108.699) (width 0.2) (layer "B.Cu") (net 8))
 (segment (start 172.979 113.689) (end 154.919 113.689) (width 0.2) (layer "F.Cu") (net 11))
 (segment (start 154.919 113.689) (end 146.19 104.96) (width 0.2) (layer "F.Cu") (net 11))
 (segment (start 174.13 114.84) (end 172.979 113.689) (width 0.2) (layer "F.Cu") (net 11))
 (segment (start 132.4 111.915) (end 139.595 104.72) (width 0.2) (layer "F.Cu") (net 6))
 (segment (start 123.4 106.4) (end 121 104) (width 0.2) (layer "F.Cu") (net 6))
 (segment (start 125.91 114.84) (end 123.4 112.33) (width 0.2) (layer "F.Cu") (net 6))
 (segment (start 127.061 115.991) (end 129.324 115.991) (width 0.2) (layer "F.Cu") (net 6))
 (segment (start 129.324 115.991) (end 132.4 112.915) (width 0.2) (layer "F.Cu") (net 6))
 (segment (start 123.4 112.33) (end 123.4 106.4) (width 0.2) (layer "F.Cu") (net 6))
 (segment (start 132.4 112.915) (end 132.4 111.915) (width 0.2) (layer "F.Cu") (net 6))
 (segment (start 139.595 104.72) (end 140.595 104.72) (width 0.2) (layer "F.Cu") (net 6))
 (segment (start 125.91 114.84) (end 127.061 115.991) (width 0.2) (layer "F.Cu") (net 6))
 (segment (start 140.595 104.72) (end 141.456 103.859) (width 0.2) (layer "B.Cu") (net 6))
 (segment (start 150.169 103.859) (end 151.27 104.96) (width 0.2) (layer "B.Cu") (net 6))
 (segment (start 141.456 103.859) (end 150.169 103.859) (width 0.2) (layer "B.Cu") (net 6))
 (segment (start 158.304 106.159) (end 159.405 107.26) (width 0.2) (layer "F.Cu") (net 4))
 (segment (start 123.211 98.211) (end 156.05305 98.211) (width 0.2) (layer "F.Cu") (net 4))
 (segment (start 156.05305 98.211) (end 158.304 100.46195) (width 0.2) (layer "F.Cu") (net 4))
 (segment (start 158.304 100.46195) (end 158.304 106.159) (width 0.2) (layer "F.Cu") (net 4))
 (segment (start 121 96) (end 123.211 98.211) (width 0.2) (layer "F.Cu") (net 4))
 (segment (start 152.54 79.15) (end 152.54 89.17) (width 0.2) (layer "F.Cu") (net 32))
 (segment (start 157.62 79.15) (end 157.62 89.17) (width 0.2) (layer "F.Cu") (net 34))
 (segment (start 147.46 79.15) (end 147.46 89.17) (width 0.2) (layer "F.Cu") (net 30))
 (segment (start 142.38 89.17) (end 142.38 79.15) (width 0.2) (layer "F.Cu") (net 28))
 (segment (start 144.92 77.5) (end 144.92 89.17) (width 0.2) (layer "F.Cu") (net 29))
 (segment (start 150 77.5) (end 150 89.17) (width 0.2) (layer "F.Cu") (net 31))
 (segment (start 155.08 77.5) (end 155.08 89.17) (width 0.2) (layer "F.Cu") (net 33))
 (segment (start 172.979 121.071) (end 154.406 121.071) (width 0.2) (layer "F.Cu") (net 27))
 (segment (start 174.13 119.92) (end 172.979 121.071) (width 0.2) (layer "F.Cu") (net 27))
 (segment (start 154.406 121.071) (end 140.595 107.26) (width 0.2) (layer "F.Cu") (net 27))
 (segment (start 126.38676 108.609) (end 127.299 109.52124) (width 0.2) (layer "F.Cu") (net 5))
 (segment (start 121 100) (end 123.801 102.801) (width 0.2) (layer "F.Cu") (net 5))
 (segment (start 123.801 102.801) (end 123.801 107.401) (width 0.2) (layer "F.Cu") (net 5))
 (segment (start 127.299 109.52124) (end 127.299 112.897) (width 0.2) (layer "F.Cu") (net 5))
 (segment (start 125.009 108.609) (end 126.38676 108.609) (width 0.2) (layer "F.Cu") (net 5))
 (segment (start 127.299 112.897) (end 128.45 114.048) (width 0.2) (layer "F.Cu") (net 5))
 (segment (start 123.801 107.401) (end 125.009 108.609) (width 0.2) (layer "F.Cu") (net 5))
 (segment (start 128.45 114.048) (end 128.45 114.84) (width 0.2) (layer "F.Cu") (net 5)))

